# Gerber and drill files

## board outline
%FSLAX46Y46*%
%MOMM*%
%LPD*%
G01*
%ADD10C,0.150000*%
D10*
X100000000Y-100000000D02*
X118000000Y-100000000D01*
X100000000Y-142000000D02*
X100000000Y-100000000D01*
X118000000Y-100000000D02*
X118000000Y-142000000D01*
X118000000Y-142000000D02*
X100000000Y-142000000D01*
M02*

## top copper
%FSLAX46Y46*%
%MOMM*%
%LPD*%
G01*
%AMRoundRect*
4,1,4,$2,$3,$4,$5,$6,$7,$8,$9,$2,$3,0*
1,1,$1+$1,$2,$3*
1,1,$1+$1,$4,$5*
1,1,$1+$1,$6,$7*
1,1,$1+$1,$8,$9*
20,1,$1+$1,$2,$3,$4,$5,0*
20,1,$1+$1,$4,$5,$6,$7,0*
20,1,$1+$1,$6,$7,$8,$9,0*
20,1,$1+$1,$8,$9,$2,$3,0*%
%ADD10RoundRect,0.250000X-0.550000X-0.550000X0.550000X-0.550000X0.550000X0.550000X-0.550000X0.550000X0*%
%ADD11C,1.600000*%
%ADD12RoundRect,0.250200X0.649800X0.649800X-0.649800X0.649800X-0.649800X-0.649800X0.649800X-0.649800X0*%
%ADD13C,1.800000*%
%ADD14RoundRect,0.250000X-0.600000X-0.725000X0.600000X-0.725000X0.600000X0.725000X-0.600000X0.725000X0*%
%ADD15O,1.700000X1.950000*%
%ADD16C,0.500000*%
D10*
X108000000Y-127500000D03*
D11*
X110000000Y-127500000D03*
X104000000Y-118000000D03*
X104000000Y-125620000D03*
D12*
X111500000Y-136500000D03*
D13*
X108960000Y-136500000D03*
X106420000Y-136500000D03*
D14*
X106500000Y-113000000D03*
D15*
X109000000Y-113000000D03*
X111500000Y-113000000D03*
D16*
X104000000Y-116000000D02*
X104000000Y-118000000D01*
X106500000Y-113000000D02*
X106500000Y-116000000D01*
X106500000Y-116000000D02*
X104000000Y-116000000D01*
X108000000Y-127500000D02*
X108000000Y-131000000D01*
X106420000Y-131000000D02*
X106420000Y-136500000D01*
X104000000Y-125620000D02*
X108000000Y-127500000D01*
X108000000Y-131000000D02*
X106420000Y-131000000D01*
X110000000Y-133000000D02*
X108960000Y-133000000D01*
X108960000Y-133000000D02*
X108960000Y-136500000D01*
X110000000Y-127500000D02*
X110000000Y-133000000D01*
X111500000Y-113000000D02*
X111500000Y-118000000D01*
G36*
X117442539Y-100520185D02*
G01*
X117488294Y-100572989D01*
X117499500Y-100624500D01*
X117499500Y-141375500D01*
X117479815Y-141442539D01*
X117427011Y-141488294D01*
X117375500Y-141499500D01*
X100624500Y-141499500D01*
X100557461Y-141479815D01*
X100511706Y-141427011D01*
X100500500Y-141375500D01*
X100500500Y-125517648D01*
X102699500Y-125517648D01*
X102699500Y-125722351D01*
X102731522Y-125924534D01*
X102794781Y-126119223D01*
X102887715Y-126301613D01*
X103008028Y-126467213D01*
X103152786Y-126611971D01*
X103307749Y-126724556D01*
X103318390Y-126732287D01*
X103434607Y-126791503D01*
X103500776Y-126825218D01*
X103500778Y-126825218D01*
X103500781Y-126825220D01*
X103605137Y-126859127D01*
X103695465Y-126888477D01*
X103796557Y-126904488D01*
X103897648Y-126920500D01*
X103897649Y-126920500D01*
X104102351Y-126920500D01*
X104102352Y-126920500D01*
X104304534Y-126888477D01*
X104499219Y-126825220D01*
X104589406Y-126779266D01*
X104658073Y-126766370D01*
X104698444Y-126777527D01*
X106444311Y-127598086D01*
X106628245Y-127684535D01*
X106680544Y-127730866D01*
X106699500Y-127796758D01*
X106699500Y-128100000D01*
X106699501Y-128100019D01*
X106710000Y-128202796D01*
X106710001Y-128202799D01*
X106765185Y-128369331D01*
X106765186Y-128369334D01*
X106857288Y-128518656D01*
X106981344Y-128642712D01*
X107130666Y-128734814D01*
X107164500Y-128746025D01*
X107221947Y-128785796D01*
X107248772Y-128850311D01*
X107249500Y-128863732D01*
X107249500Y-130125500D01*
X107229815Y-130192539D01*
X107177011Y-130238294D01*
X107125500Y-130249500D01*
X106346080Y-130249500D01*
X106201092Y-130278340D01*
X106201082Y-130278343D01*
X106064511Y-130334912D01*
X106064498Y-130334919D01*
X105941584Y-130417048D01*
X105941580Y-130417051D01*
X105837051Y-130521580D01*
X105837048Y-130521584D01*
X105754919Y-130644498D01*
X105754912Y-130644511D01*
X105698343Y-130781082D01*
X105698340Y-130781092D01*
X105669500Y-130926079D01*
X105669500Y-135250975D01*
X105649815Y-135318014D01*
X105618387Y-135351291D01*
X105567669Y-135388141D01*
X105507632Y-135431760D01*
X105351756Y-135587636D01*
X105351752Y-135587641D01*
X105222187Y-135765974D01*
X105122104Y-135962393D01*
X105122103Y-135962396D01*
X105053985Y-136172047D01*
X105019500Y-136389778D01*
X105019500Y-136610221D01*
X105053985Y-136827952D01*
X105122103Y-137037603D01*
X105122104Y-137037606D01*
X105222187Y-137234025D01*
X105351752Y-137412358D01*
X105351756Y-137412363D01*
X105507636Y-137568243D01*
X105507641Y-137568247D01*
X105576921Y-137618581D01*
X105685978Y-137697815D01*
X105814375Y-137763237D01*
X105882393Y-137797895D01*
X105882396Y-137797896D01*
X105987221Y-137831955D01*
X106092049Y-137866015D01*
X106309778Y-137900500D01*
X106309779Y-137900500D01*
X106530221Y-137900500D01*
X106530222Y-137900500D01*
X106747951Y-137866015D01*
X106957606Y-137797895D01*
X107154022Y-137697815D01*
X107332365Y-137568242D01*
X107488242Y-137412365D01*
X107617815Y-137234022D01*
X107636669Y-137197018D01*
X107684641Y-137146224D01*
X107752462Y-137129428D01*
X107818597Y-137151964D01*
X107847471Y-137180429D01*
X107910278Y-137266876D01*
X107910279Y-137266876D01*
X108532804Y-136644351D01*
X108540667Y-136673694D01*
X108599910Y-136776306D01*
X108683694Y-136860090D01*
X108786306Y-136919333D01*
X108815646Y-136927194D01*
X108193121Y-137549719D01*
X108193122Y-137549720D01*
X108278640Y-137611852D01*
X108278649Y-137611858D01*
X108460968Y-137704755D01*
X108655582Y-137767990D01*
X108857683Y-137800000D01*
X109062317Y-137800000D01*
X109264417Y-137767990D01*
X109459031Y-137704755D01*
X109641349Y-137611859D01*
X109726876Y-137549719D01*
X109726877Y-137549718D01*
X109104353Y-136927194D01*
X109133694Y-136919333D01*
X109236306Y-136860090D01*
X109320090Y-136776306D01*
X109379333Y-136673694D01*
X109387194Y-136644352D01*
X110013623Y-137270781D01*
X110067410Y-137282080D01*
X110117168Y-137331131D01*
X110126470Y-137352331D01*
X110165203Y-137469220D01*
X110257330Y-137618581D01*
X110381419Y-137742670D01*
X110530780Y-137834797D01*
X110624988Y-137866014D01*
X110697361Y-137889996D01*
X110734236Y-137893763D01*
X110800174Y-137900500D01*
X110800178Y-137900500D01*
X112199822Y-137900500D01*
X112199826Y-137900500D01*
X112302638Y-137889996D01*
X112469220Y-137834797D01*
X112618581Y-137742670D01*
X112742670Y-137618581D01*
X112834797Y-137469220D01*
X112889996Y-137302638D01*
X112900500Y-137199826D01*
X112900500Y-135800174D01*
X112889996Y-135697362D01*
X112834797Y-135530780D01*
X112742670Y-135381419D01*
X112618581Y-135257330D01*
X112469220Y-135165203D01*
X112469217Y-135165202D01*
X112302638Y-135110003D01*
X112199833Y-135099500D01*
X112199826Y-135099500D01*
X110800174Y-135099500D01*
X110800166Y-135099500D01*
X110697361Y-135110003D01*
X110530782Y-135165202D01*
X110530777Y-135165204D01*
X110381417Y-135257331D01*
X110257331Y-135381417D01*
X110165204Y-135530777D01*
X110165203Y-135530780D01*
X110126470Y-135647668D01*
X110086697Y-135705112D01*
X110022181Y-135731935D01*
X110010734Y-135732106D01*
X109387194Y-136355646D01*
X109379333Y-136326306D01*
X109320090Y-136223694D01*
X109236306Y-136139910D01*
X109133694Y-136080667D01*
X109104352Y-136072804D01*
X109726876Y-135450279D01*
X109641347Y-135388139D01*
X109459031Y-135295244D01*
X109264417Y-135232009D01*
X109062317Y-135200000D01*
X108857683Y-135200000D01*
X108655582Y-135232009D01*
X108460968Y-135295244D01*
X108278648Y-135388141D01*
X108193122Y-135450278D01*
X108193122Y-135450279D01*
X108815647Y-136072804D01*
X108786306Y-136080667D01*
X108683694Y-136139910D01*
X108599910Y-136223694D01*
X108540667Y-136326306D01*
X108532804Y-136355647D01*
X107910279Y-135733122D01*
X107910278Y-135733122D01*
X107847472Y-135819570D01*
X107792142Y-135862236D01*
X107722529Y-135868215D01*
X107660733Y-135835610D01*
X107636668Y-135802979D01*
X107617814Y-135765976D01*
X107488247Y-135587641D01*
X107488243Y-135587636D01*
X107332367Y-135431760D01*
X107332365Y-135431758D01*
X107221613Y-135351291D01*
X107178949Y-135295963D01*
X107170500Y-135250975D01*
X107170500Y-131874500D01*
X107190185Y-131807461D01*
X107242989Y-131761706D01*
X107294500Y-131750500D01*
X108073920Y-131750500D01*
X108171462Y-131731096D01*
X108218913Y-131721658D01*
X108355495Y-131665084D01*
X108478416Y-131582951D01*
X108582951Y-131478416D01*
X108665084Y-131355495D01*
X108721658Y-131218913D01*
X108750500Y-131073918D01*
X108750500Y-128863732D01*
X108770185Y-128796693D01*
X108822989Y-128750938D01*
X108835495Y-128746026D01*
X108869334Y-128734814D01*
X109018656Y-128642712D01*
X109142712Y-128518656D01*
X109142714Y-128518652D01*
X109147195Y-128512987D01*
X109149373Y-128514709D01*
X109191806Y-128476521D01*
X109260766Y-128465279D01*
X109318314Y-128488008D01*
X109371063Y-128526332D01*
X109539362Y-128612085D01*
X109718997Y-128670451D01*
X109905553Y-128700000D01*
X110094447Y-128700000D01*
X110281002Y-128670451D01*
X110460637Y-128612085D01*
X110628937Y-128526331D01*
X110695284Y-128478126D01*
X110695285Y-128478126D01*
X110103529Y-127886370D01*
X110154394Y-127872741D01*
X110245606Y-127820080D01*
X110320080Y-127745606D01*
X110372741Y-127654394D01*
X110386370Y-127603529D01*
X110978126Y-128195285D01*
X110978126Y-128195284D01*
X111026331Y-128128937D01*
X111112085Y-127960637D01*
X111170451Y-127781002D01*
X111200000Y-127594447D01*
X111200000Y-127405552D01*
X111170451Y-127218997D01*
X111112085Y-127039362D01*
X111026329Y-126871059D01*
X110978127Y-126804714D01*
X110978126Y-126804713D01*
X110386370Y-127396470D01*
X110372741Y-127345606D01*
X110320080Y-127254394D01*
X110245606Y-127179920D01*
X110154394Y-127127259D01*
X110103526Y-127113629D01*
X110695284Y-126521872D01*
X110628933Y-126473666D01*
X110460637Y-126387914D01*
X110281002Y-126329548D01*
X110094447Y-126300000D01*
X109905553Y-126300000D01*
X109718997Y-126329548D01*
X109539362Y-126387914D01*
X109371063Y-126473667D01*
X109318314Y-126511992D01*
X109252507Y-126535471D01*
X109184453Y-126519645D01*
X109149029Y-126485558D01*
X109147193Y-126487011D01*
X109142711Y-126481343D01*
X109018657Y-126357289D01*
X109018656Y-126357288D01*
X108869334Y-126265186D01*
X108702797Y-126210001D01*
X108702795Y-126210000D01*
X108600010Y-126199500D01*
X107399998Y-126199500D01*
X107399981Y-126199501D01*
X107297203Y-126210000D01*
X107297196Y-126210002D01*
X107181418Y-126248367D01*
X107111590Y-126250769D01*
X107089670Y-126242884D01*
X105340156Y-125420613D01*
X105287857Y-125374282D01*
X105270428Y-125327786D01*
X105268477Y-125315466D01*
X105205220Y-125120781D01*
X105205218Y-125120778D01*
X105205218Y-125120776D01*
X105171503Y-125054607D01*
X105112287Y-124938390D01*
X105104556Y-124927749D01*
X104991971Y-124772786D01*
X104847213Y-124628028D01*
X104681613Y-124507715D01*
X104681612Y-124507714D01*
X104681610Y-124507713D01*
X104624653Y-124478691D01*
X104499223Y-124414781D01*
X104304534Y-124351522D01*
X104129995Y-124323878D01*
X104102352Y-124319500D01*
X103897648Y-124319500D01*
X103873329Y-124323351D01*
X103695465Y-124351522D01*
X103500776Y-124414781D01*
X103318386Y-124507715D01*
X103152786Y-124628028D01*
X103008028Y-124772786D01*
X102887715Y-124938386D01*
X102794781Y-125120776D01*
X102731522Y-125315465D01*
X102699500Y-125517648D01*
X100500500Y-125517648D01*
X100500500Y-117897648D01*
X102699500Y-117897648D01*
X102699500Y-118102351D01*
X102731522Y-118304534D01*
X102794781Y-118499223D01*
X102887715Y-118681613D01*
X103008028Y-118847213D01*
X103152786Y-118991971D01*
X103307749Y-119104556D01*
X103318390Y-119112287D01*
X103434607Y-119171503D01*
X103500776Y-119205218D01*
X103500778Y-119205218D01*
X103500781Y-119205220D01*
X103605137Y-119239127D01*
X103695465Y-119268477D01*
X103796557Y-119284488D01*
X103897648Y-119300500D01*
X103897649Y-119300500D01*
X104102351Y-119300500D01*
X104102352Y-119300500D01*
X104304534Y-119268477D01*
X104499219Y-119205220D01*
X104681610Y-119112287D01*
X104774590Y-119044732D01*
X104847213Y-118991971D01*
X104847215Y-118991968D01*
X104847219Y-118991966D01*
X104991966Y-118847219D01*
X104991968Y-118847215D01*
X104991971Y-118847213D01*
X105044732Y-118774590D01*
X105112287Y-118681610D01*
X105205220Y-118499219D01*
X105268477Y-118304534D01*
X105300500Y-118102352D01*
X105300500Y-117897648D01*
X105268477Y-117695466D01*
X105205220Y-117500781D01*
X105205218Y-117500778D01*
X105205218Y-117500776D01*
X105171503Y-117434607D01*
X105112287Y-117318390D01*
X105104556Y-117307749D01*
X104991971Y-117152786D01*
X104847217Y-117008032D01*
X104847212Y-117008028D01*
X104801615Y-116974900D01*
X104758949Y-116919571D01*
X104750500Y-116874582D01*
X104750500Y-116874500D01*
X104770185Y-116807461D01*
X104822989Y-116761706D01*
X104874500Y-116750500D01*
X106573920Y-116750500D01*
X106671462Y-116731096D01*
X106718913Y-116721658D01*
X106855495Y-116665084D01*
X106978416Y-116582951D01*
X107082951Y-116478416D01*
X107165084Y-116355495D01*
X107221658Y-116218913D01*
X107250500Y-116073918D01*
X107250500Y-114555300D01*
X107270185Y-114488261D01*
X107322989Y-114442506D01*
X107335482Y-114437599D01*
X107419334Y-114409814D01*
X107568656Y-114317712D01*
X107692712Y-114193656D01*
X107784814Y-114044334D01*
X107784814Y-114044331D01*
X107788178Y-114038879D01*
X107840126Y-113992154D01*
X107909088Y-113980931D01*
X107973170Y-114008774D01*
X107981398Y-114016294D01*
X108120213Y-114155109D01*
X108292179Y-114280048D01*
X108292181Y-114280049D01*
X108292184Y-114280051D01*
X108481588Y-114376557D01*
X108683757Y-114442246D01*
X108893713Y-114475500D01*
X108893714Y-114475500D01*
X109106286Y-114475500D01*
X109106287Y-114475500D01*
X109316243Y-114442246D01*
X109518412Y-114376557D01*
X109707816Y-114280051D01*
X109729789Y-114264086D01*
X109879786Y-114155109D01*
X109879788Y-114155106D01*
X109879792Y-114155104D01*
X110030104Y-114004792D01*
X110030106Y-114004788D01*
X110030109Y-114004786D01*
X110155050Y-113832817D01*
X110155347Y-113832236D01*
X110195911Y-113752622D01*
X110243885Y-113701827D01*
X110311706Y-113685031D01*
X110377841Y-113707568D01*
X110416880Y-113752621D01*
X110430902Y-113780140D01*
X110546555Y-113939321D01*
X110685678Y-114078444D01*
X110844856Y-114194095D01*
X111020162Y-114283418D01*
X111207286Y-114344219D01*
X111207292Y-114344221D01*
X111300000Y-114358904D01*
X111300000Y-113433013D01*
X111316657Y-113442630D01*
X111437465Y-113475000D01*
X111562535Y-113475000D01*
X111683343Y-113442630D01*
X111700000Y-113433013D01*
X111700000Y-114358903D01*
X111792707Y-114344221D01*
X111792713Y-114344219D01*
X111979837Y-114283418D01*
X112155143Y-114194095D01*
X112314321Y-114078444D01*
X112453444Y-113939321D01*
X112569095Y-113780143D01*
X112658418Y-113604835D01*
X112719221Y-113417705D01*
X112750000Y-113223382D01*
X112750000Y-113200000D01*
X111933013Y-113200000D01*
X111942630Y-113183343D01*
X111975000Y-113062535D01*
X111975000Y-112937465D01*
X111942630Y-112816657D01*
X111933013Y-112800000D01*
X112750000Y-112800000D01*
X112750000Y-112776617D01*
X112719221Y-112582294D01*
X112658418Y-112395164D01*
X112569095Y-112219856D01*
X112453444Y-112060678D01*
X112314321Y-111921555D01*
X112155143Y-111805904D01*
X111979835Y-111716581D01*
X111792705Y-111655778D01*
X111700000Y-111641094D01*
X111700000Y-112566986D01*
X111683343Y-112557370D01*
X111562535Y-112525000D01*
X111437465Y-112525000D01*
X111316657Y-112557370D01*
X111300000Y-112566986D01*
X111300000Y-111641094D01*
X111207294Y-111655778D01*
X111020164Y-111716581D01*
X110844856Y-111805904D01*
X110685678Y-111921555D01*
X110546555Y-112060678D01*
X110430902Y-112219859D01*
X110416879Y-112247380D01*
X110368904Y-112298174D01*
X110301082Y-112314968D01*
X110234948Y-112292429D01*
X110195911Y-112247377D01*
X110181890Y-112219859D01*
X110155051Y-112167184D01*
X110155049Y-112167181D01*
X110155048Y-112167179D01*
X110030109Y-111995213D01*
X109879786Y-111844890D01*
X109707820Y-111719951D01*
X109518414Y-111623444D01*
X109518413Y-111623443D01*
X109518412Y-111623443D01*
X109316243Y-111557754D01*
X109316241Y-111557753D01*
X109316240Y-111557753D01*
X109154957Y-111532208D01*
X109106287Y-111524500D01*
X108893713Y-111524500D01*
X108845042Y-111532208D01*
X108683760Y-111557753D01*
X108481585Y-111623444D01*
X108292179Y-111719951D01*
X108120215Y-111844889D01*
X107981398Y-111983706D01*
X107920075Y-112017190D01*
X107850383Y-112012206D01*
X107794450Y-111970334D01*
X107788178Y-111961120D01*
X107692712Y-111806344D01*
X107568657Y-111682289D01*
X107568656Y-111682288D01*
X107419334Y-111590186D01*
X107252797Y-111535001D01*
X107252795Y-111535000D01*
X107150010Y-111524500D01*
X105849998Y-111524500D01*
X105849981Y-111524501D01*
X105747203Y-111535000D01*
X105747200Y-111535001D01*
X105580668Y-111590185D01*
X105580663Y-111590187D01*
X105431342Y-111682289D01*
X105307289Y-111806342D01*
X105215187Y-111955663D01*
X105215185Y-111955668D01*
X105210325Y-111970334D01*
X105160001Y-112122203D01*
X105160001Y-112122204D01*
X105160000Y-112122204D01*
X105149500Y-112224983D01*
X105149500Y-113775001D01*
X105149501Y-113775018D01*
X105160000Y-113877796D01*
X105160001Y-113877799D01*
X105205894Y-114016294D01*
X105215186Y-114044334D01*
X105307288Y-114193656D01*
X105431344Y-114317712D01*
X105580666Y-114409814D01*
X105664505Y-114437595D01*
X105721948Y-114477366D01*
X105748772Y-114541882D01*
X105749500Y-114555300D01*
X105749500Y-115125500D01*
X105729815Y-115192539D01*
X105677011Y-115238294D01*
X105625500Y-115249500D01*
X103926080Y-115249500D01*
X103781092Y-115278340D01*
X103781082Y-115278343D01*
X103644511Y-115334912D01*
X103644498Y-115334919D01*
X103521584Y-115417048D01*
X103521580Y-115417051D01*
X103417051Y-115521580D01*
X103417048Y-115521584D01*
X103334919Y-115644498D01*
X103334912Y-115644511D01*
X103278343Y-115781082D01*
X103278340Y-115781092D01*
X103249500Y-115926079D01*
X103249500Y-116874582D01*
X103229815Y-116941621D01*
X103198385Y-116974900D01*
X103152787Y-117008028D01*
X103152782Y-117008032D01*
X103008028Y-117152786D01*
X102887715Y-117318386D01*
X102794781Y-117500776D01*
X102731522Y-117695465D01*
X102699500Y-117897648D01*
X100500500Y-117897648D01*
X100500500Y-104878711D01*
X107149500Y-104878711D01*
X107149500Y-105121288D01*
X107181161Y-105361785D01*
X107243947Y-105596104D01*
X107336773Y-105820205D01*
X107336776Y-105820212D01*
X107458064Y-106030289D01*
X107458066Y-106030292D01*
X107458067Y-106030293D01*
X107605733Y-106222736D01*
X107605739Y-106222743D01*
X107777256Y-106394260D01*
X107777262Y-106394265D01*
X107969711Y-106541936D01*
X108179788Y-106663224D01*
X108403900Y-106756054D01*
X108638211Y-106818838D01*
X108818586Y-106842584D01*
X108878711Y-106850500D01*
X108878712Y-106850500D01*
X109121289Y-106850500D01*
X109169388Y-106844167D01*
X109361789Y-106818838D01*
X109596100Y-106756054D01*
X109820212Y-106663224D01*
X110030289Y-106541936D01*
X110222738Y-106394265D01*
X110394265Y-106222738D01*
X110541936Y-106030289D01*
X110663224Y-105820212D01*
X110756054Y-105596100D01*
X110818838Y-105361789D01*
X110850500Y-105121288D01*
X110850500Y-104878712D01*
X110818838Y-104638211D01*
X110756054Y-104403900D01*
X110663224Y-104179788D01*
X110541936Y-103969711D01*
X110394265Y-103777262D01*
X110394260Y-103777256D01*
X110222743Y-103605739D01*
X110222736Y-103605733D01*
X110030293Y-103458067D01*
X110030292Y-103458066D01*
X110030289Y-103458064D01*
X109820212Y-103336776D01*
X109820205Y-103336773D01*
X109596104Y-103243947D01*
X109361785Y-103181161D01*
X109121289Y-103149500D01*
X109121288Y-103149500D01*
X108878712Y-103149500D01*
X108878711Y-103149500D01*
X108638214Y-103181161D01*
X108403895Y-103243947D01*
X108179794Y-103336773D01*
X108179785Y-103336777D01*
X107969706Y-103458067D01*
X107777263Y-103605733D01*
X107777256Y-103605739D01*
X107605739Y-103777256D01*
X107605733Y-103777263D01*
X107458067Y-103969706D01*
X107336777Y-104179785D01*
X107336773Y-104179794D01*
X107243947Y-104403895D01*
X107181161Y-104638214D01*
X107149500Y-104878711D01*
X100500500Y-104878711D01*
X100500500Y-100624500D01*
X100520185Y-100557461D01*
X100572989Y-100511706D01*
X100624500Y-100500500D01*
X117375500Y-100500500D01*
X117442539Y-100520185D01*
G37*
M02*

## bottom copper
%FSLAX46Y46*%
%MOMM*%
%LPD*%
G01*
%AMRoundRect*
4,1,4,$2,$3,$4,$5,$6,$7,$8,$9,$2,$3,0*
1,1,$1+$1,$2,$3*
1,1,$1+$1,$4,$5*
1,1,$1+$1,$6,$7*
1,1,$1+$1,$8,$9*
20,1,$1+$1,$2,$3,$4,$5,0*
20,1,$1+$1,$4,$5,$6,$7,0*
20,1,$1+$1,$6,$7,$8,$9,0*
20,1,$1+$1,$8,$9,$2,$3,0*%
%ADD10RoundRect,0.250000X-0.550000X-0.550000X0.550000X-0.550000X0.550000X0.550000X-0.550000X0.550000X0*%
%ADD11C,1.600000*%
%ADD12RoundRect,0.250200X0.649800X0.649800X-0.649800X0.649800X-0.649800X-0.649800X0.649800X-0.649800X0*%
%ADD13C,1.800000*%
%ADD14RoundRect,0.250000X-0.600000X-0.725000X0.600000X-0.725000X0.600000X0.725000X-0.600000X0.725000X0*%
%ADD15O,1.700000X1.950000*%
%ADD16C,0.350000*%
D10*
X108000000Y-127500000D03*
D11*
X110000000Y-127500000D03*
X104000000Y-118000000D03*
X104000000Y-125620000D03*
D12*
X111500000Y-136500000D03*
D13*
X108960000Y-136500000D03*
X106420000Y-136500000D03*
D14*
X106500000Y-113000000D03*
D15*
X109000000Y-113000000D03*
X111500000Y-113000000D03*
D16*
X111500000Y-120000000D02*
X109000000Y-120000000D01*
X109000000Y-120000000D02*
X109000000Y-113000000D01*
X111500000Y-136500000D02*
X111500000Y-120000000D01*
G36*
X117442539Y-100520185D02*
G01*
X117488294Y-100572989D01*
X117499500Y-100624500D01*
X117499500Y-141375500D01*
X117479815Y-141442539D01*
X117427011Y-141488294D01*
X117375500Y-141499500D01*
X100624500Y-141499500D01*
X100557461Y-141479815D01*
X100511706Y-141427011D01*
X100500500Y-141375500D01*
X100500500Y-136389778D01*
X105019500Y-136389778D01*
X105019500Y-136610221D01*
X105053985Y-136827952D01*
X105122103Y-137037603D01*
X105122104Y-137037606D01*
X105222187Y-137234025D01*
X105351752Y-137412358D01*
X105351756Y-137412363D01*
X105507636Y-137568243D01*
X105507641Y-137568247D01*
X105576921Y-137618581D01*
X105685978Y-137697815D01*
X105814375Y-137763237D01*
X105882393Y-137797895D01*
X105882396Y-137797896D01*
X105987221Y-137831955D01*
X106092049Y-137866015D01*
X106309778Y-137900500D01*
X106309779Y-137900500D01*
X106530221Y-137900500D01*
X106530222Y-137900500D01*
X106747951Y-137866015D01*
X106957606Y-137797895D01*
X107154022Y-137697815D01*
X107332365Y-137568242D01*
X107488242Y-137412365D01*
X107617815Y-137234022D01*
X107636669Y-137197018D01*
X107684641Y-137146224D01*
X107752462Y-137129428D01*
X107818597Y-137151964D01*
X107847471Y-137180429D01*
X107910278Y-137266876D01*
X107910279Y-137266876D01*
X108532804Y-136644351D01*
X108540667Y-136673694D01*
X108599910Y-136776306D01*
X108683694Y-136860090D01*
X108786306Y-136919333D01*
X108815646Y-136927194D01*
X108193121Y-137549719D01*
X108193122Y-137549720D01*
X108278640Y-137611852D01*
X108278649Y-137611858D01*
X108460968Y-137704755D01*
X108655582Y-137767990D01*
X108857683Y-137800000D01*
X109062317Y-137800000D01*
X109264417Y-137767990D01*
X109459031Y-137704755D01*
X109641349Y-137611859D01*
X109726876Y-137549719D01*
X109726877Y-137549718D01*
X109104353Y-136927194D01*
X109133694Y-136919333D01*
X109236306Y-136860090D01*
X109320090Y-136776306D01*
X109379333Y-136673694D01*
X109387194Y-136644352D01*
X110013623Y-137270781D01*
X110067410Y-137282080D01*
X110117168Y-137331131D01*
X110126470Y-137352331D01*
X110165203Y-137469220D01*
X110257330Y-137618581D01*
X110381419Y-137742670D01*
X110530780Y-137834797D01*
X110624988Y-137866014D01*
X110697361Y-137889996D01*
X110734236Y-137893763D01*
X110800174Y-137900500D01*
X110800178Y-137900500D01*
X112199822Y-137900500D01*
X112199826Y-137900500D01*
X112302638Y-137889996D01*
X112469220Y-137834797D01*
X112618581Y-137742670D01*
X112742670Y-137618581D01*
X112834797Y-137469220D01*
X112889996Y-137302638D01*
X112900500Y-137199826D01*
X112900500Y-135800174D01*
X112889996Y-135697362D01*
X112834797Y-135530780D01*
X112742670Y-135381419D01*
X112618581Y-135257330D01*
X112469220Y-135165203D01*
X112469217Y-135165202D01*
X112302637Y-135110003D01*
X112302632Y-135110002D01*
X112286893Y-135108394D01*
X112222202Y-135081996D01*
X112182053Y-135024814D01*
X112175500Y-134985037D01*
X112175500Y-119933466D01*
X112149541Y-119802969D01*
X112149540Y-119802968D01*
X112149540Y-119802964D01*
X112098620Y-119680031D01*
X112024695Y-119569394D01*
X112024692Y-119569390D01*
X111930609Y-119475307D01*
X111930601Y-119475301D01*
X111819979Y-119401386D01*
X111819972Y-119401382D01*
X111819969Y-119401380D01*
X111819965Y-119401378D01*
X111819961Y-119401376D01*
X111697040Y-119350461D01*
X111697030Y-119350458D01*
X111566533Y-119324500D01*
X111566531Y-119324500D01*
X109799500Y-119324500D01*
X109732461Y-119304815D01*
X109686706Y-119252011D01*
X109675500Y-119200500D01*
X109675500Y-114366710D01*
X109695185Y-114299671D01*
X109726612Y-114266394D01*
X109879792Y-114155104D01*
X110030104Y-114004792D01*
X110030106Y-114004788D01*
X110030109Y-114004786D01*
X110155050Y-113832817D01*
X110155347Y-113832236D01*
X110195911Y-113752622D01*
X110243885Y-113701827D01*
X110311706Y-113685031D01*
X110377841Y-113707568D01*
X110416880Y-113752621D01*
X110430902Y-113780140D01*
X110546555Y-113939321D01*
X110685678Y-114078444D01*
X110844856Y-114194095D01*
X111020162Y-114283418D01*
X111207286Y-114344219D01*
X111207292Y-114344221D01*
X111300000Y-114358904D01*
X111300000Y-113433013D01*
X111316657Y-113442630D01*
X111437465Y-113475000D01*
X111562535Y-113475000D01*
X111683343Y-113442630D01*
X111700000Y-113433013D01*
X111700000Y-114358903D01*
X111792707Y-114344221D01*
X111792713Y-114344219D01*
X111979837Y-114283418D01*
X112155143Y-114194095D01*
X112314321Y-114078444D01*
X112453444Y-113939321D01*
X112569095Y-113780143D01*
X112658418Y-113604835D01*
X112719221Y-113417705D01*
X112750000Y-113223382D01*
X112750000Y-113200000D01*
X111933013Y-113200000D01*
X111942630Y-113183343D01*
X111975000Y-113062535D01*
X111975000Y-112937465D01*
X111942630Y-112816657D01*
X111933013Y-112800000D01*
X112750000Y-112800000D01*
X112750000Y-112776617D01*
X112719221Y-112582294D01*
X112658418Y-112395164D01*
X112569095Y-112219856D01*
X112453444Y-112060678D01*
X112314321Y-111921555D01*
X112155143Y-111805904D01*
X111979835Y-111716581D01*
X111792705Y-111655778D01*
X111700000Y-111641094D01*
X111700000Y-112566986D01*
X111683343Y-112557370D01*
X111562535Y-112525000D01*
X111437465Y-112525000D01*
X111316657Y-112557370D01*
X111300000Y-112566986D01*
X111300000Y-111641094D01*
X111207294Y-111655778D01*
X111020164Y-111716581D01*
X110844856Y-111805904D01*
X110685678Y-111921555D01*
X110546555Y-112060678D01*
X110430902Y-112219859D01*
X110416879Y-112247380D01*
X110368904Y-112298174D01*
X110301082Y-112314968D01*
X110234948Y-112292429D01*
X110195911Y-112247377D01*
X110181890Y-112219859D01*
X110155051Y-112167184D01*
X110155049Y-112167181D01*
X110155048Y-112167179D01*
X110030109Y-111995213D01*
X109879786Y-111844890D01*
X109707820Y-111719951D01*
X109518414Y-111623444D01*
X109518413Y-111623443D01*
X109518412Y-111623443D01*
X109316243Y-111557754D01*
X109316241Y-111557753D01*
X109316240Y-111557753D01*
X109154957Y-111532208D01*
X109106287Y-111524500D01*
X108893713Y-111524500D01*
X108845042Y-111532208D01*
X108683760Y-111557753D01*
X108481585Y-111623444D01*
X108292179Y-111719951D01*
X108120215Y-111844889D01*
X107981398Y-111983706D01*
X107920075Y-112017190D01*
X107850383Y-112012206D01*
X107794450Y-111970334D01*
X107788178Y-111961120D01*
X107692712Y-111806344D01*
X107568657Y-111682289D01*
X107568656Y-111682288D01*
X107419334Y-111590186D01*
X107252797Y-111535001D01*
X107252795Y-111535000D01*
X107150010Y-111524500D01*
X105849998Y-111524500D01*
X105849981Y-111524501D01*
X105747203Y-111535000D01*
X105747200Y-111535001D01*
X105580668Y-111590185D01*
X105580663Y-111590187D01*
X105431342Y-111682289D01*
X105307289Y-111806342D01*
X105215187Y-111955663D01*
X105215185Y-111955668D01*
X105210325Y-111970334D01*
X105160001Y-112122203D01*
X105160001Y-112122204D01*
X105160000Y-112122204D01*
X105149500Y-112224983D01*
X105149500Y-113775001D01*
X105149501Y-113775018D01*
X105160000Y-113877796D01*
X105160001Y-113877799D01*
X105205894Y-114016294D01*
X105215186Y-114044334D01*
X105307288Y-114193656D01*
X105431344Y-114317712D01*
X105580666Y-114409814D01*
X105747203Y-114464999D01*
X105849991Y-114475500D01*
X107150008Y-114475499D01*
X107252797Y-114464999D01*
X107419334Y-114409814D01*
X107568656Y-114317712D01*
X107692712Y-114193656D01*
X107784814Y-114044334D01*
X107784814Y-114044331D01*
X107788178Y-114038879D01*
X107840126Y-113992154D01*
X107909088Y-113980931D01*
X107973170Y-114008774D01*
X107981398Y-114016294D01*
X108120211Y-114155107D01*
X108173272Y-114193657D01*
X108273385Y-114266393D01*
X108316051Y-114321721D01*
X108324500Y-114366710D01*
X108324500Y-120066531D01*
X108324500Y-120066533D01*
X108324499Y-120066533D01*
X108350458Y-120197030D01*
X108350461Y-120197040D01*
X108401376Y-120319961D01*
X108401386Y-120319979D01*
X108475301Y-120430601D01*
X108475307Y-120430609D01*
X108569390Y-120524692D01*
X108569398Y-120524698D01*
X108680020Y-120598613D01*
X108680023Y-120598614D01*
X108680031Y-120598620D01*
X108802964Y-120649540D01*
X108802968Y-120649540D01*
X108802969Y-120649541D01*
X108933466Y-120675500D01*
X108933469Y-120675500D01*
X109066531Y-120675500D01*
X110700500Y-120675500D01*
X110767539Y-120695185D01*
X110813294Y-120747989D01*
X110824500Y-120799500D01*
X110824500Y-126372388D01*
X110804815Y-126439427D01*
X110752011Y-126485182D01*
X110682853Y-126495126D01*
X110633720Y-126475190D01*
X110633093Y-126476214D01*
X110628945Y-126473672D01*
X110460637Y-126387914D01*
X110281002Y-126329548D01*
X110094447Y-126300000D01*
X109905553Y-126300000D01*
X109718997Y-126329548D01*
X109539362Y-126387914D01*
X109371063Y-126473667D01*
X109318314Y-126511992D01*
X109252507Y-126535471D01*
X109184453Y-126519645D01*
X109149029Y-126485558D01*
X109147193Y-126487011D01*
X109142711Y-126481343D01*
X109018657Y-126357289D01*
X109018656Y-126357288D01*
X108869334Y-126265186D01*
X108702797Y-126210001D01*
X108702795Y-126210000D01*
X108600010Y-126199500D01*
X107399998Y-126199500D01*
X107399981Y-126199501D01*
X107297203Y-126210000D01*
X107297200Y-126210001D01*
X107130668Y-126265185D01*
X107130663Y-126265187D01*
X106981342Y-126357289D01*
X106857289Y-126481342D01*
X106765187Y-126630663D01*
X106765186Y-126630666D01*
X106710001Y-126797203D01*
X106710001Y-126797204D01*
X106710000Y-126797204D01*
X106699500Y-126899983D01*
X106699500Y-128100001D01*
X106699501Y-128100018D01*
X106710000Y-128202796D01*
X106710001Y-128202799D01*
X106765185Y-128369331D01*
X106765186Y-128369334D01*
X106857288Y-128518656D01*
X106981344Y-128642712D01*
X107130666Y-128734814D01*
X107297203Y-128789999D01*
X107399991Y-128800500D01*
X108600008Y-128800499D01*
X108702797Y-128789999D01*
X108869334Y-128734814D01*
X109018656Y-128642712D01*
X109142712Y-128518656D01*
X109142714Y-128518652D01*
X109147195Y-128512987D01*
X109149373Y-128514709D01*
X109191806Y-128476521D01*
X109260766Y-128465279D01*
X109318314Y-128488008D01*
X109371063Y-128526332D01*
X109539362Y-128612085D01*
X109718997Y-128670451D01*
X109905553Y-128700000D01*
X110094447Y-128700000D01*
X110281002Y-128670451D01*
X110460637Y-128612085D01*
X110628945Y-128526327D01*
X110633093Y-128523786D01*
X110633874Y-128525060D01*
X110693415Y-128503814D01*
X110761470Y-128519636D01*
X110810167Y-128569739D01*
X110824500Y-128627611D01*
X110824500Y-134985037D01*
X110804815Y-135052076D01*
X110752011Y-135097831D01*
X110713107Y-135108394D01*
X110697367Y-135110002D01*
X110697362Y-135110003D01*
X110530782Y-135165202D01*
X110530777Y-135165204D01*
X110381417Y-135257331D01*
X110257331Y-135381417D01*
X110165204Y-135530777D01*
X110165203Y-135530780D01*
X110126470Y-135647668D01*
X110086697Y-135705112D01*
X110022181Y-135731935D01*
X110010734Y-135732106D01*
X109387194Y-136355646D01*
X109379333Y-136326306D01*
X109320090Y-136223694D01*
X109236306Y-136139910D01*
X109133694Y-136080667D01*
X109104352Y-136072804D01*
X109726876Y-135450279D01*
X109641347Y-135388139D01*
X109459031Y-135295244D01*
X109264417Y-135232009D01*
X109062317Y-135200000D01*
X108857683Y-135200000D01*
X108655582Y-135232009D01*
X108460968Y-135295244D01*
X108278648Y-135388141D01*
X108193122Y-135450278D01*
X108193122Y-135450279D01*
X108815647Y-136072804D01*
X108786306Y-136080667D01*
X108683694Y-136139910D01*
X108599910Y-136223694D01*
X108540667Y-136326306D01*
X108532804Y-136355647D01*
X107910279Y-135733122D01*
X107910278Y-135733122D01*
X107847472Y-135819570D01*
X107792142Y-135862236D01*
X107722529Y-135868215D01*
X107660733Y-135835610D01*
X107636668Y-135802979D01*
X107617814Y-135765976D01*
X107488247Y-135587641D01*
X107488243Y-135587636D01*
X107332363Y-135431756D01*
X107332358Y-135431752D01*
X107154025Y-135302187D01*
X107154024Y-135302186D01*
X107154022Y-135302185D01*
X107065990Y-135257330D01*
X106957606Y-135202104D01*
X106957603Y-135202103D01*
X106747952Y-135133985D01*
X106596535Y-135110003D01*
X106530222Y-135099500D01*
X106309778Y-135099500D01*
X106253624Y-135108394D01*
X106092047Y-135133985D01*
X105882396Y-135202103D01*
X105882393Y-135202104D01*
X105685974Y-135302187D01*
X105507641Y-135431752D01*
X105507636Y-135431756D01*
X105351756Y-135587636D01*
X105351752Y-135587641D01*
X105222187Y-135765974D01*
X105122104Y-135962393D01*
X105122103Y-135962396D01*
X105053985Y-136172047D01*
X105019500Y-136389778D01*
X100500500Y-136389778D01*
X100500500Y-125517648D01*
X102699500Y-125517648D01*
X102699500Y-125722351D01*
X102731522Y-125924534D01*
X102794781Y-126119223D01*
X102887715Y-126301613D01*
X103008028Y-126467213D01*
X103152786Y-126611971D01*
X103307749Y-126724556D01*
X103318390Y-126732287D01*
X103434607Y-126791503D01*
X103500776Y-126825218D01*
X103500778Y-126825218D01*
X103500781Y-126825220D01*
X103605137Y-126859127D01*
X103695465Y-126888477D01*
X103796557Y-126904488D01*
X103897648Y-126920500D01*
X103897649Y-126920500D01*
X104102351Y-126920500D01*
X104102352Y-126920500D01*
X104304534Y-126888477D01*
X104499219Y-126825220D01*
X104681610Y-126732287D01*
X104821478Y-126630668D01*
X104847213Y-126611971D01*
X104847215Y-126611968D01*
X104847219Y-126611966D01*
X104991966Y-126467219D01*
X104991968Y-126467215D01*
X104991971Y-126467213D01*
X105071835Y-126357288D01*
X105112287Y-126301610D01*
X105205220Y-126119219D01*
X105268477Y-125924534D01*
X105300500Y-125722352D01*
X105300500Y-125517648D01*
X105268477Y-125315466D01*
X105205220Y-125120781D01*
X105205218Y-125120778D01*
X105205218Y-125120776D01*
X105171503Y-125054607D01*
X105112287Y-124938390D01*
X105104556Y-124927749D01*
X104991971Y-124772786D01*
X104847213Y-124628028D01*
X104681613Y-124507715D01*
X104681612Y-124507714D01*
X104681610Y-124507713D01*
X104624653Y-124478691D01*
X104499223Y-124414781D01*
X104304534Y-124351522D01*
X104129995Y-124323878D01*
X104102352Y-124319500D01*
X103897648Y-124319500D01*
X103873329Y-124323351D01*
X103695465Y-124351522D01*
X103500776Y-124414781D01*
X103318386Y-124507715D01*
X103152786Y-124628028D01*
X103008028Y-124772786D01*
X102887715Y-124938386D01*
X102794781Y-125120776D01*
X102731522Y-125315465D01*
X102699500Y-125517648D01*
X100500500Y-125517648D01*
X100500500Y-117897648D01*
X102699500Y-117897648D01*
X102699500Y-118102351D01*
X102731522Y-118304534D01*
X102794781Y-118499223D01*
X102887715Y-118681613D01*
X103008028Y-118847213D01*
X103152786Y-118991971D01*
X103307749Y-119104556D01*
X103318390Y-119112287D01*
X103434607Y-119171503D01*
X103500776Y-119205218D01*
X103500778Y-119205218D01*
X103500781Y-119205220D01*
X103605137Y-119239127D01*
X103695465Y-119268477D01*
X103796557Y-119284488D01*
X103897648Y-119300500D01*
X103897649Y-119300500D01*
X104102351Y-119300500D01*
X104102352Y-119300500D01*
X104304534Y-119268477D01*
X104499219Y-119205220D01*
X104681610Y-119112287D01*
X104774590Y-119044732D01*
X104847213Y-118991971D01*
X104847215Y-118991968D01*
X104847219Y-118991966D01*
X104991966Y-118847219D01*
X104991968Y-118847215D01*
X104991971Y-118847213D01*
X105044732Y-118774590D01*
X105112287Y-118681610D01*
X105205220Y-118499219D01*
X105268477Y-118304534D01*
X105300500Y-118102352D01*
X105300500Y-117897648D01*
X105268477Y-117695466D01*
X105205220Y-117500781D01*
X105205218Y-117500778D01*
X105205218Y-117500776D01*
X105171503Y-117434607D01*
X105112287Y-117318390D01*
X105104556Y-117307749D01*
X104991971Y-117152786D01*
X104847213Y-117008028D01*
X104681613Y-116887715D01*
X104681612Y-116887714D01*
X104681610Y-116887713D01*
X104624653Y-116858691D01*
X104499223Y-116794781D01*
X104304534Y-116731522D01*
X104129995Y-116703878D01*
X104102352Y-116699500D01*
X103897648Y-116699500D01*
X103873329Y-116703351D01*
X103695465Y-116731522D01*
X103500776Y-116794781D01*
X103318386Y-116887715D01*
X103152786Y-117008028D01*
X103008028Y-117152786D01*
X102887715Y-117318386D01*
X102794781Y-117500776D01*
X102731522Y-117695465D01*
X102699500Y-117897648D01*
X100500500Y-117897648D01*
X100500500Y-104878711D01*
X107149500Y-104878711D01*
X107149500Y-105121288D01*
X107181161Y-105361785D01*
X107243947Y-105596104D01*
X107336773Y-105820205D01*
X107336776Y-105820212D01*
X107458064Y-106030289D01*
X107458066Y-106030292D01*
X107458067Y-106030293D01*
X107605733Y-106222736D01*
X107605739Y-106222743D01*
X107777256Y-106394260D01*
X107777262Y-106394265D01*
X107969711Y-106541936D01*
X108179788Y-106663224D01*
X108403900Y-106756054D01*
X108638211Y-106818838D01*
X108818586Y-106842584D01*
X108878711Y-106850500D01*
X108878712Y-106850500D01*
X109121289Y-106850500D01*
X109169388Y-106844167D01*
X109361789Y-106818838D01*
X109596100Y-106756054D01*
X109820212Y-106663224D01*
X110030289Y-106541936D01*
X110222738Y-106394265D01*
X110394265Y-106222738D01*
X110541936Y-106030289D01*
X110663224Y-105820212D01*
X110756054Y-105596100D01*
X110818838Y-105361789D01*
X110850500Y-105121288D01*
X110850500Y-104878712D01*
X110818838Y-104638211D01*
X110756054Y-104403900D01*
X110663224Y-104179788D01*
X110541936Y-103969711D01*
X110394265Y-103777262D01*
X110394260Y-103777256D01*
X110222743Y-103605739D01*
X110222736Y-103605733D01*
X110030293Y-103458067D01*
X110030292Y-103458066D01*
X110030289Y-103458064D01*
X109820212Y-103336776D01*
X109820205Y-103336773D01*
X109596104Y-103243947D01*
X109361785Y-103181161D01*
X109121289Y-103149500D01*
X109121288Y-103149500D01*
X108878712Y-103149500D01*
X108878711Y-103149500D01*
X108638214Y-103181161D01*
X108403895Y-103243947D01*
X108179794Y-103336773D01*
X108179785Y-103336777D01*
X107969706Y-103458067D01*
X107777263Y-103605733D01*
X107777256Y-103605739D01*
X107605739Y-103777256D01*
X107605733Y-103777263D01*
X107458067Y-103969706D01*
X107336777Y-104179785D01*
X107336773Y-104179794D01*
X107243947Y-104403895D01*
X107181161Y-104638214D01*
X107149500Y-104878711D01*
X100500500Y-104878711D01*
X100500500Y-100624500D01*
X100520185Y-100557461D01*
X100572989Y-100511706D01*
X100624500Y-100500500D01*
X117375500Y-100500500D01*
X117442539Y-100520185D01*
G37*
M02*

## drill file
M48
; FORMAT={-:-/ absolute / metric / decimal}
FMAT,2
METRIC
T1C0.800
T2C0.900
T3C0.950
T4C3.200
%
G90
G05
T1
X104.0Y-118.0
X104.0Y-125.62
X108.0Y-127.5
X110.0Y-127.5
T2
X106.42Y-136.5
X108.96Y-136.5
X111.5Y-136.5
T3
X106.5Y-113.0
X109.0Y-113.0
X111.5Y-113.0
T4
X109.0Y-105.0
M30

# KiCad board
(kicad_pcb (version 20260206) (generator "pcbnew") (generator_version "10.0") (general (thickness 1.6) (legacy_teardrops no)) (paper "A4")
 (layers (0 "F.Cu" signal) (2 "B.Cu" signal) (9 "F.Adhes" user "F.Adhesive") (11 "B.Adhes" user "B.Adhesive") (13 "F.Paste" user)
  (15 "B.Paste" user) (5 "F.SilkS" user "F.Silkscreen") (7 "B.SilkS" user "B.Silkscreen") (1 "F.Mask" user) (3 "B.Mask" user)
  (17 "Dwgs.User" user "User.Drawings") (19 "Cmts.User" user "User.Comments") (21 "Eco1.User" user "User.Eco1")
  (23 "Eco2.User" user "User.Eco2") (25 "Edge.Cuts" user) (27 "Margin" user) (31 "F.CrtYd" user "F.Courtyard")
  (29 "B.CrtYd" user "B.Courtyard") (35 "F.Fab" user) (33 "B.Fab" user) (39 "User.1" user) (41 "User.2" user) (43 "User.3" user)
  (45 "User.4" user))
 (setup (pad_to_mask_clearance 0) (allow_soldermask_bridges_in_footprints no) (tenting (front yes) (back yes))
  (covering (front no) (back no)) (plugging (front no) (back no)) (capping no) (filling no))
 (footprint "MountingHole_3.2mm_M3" (layer "F.Cu") (at 109 105)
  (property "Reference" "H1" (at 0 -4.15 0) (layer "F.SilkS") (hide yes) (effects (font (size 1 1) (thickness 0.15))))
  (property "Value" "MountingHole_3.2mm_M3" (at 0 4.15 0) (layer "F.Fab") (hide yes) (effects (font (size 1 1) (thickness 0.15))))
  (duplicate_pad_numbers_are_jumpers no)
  (pad "" np_thru_hole circle (at 0 0) (size 3.2 3.2) (drill 3.2) (layers "*.Cu" "*.Mask")))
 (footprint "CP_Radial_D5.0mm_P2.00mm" (layer "F.Cu") (at 108 127.5)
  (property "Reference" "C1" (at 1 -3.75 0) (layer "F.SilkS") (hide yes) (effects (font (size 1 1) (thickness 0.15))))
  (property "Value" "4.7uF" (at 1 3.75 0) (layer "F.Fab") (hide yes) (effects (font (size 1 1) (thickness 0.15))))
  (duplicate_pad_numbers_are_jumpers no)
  (pad "1" thru_hole roundrect (at 0 0) (size 1.6 1.6) (drill 0.8) (layers "*.Cu" "*.Mask") (remove_unused_layers no)
   (roundrect_rratio 0.15625) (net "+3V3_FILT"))
  (pad "2" thru_hole circle (at 2 0) (size 1.6 1.6) (drill 0.8) (layers "*.Cu" "*.Mask") (remove_unused_layers no) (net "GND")))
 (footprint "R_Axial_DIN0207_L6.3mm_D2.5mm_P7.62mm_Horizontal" (layer "F.Cu") (at 104 118 -90)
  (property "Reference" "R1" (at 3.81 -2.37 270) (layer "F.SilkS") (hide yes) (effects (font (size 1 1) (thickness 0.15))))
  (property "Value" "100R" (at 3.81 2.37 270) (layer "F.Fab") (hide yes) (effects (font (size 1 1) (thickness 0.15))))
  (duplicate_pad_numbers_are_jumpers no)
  (pad "1" thru_hole circle (at 0 0 270) (size 1.6 1.6) (drill 0.8) (layers "*.Cu" "*.Mask") (remove_unused_layers no) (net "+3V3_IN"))
  (pad "2" thru_hole circle (at 7.62 0 270) (size 1.6 1.6) (drill 0.8) (layers "*.Cu" "*.Mask") (remove_unused_layers no) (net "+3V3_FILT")))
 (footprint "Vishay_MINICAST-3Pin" (layer "F.Cu") (at 111.5 136.5 180)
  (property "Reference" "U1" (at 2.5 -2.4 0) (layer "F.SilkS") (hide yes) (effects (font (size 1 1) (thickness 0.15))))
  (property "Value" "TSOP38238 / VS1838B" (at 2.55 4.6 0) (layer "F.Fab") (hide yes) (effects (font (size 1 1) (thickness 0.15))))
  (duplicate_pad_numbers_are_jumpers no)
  (pad "1" thru_hole roundrect (at 0 0 180) (size 1.8 1.8) (drill 0.9) (layers "*.Cu" "*.Mask") (remove_unused_layers no)
   (roundrect_rratio 0.139) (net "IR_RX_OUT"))
  (pad "2" thru_hole circle (at 2.54 0 180) (size 1.8 1.8) (drill 0.9) (layers "*.Cu" "*.Mask") (remove_unused_layers no) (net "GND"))
  (pad "3" thru_hole circle (at 5.08 0 180) (size 1.8 1.8) (drill 0.9) (layers "*.Cu" "*.Mask") (remove_unused_layers no) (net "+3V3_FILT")))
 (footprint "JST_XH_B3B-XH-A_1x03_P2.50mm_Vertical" (layer "F.Cu") (at 106.5 113)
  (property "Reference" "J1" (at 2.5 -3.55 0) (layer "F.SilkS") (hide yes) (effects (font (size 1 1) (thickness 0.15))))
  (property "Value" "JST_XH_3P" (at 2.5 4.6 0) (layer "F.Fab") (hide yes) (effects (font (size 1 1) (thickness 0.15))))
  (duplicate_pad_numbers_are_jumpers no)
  (pad "1" thru_hole roundrect (at 0 0) (size 1.7 1.95) (drill 0.95) (layers "*.Cu" "*.Mask") (remove_unused_layers no)
   (roundrect_rratio 0.147059) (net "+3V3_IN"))
  (pad "2" thru_hole oval (at 2.5 0) (size 1.7 1.95) (drill 0.95) (layers "*.Cu" "*.Mask") (remove_unused_layers no) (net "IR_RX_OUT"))
  (pad "3" thru_hole oval (at 5 0) (size 1.7 1.95) (drill 0.95) (layers "*.Cu" "*.Mask") (remove_unused_layers no) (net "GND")))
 (gr_line (start 100 100) (end 118 100) (stroke (width 0.15) (type default)) (layer "Edge.Cuts"))
 (gr_line (start 100 142) (end 100 100) (stroke (width 0.15) (type default)) (layer "Edge.Cuts"))
 (gr_line (start 118 100) (end 118 142) (stroke (width 0.15) (type default)) (layer "Edge.Cuts"))
 (gr_line (start 118 142) (end 100 142) (stroke (width 0.15) (type default)) (layer "Edge.Cuts"))
 (segment (start 104 116) (end 104 118) (width 0.5) (layer "F.Cu") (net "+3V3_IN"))
 (segment (start 106.5 113) (end 106.5 116) (width 0.5) (layer "F.Cu") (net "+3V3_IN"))
 (segment (start 106.5 116) (end 104 116) (width 0.5) (layer "F.Cu") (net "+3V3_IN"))
 (segment (start 108 127.5) (end 108 131) (width 0.5) (layer "F.Cu") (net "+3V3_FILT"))
 (segment (start 106.42 131) (end 106.42 136.5) (width 0.5) (layer "F.Cu") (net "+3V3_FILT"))
 (segment (start 104 125.62) (end 108 127.5) (width 0.5) (layer "F.Cu") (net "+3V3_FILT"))
 (segment (start 108 131) (end 106.42 131) (width 0.5) (layer "F.Cu") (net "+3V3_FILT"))
 (segment (start 111.5 120) (end 109 120) (width 0.35) (layer "B.Cu") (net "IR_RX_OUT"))
 (segment (start 109 120) (end 109 113) (width 0.35) (layer "B.Cu") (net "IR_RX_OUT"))
 (segment (start 111.5 136.5) (end 111.5 120) (width 0.35) (layer "B.Cu") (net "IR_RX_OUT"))
 (segment (start 110 133) (end 108.96 133) (width 0.5) (layer "F.Cu") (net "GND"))
 (segment (start 108.96 133) (end 108.96 136.5) (width 0.5) (layer "F.Cu") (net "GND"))
 (segment (start 110 127.5) (end 110 133) (width 0.5) (layer "F.Cu") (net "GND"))
 (segment (start 111.5 113) (end 111.5 118) (width 0.5) (layer "F.Cu") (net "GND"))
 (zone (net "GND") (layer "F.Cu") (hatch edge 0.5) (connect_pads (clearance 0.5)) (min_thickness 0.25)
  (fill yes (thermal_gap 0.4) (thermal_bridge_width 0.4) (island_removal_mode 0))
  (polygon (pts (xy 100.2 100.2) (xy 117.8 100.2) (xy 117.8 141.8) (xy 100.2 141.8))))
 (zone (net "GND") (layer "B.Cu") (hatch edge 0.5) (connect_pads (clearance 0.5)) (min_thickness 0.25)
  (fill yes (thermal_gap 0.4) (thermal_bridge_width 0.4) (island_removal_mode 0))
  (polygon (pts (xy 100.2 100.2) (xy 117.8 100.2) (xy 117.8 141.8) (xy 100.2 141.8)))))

